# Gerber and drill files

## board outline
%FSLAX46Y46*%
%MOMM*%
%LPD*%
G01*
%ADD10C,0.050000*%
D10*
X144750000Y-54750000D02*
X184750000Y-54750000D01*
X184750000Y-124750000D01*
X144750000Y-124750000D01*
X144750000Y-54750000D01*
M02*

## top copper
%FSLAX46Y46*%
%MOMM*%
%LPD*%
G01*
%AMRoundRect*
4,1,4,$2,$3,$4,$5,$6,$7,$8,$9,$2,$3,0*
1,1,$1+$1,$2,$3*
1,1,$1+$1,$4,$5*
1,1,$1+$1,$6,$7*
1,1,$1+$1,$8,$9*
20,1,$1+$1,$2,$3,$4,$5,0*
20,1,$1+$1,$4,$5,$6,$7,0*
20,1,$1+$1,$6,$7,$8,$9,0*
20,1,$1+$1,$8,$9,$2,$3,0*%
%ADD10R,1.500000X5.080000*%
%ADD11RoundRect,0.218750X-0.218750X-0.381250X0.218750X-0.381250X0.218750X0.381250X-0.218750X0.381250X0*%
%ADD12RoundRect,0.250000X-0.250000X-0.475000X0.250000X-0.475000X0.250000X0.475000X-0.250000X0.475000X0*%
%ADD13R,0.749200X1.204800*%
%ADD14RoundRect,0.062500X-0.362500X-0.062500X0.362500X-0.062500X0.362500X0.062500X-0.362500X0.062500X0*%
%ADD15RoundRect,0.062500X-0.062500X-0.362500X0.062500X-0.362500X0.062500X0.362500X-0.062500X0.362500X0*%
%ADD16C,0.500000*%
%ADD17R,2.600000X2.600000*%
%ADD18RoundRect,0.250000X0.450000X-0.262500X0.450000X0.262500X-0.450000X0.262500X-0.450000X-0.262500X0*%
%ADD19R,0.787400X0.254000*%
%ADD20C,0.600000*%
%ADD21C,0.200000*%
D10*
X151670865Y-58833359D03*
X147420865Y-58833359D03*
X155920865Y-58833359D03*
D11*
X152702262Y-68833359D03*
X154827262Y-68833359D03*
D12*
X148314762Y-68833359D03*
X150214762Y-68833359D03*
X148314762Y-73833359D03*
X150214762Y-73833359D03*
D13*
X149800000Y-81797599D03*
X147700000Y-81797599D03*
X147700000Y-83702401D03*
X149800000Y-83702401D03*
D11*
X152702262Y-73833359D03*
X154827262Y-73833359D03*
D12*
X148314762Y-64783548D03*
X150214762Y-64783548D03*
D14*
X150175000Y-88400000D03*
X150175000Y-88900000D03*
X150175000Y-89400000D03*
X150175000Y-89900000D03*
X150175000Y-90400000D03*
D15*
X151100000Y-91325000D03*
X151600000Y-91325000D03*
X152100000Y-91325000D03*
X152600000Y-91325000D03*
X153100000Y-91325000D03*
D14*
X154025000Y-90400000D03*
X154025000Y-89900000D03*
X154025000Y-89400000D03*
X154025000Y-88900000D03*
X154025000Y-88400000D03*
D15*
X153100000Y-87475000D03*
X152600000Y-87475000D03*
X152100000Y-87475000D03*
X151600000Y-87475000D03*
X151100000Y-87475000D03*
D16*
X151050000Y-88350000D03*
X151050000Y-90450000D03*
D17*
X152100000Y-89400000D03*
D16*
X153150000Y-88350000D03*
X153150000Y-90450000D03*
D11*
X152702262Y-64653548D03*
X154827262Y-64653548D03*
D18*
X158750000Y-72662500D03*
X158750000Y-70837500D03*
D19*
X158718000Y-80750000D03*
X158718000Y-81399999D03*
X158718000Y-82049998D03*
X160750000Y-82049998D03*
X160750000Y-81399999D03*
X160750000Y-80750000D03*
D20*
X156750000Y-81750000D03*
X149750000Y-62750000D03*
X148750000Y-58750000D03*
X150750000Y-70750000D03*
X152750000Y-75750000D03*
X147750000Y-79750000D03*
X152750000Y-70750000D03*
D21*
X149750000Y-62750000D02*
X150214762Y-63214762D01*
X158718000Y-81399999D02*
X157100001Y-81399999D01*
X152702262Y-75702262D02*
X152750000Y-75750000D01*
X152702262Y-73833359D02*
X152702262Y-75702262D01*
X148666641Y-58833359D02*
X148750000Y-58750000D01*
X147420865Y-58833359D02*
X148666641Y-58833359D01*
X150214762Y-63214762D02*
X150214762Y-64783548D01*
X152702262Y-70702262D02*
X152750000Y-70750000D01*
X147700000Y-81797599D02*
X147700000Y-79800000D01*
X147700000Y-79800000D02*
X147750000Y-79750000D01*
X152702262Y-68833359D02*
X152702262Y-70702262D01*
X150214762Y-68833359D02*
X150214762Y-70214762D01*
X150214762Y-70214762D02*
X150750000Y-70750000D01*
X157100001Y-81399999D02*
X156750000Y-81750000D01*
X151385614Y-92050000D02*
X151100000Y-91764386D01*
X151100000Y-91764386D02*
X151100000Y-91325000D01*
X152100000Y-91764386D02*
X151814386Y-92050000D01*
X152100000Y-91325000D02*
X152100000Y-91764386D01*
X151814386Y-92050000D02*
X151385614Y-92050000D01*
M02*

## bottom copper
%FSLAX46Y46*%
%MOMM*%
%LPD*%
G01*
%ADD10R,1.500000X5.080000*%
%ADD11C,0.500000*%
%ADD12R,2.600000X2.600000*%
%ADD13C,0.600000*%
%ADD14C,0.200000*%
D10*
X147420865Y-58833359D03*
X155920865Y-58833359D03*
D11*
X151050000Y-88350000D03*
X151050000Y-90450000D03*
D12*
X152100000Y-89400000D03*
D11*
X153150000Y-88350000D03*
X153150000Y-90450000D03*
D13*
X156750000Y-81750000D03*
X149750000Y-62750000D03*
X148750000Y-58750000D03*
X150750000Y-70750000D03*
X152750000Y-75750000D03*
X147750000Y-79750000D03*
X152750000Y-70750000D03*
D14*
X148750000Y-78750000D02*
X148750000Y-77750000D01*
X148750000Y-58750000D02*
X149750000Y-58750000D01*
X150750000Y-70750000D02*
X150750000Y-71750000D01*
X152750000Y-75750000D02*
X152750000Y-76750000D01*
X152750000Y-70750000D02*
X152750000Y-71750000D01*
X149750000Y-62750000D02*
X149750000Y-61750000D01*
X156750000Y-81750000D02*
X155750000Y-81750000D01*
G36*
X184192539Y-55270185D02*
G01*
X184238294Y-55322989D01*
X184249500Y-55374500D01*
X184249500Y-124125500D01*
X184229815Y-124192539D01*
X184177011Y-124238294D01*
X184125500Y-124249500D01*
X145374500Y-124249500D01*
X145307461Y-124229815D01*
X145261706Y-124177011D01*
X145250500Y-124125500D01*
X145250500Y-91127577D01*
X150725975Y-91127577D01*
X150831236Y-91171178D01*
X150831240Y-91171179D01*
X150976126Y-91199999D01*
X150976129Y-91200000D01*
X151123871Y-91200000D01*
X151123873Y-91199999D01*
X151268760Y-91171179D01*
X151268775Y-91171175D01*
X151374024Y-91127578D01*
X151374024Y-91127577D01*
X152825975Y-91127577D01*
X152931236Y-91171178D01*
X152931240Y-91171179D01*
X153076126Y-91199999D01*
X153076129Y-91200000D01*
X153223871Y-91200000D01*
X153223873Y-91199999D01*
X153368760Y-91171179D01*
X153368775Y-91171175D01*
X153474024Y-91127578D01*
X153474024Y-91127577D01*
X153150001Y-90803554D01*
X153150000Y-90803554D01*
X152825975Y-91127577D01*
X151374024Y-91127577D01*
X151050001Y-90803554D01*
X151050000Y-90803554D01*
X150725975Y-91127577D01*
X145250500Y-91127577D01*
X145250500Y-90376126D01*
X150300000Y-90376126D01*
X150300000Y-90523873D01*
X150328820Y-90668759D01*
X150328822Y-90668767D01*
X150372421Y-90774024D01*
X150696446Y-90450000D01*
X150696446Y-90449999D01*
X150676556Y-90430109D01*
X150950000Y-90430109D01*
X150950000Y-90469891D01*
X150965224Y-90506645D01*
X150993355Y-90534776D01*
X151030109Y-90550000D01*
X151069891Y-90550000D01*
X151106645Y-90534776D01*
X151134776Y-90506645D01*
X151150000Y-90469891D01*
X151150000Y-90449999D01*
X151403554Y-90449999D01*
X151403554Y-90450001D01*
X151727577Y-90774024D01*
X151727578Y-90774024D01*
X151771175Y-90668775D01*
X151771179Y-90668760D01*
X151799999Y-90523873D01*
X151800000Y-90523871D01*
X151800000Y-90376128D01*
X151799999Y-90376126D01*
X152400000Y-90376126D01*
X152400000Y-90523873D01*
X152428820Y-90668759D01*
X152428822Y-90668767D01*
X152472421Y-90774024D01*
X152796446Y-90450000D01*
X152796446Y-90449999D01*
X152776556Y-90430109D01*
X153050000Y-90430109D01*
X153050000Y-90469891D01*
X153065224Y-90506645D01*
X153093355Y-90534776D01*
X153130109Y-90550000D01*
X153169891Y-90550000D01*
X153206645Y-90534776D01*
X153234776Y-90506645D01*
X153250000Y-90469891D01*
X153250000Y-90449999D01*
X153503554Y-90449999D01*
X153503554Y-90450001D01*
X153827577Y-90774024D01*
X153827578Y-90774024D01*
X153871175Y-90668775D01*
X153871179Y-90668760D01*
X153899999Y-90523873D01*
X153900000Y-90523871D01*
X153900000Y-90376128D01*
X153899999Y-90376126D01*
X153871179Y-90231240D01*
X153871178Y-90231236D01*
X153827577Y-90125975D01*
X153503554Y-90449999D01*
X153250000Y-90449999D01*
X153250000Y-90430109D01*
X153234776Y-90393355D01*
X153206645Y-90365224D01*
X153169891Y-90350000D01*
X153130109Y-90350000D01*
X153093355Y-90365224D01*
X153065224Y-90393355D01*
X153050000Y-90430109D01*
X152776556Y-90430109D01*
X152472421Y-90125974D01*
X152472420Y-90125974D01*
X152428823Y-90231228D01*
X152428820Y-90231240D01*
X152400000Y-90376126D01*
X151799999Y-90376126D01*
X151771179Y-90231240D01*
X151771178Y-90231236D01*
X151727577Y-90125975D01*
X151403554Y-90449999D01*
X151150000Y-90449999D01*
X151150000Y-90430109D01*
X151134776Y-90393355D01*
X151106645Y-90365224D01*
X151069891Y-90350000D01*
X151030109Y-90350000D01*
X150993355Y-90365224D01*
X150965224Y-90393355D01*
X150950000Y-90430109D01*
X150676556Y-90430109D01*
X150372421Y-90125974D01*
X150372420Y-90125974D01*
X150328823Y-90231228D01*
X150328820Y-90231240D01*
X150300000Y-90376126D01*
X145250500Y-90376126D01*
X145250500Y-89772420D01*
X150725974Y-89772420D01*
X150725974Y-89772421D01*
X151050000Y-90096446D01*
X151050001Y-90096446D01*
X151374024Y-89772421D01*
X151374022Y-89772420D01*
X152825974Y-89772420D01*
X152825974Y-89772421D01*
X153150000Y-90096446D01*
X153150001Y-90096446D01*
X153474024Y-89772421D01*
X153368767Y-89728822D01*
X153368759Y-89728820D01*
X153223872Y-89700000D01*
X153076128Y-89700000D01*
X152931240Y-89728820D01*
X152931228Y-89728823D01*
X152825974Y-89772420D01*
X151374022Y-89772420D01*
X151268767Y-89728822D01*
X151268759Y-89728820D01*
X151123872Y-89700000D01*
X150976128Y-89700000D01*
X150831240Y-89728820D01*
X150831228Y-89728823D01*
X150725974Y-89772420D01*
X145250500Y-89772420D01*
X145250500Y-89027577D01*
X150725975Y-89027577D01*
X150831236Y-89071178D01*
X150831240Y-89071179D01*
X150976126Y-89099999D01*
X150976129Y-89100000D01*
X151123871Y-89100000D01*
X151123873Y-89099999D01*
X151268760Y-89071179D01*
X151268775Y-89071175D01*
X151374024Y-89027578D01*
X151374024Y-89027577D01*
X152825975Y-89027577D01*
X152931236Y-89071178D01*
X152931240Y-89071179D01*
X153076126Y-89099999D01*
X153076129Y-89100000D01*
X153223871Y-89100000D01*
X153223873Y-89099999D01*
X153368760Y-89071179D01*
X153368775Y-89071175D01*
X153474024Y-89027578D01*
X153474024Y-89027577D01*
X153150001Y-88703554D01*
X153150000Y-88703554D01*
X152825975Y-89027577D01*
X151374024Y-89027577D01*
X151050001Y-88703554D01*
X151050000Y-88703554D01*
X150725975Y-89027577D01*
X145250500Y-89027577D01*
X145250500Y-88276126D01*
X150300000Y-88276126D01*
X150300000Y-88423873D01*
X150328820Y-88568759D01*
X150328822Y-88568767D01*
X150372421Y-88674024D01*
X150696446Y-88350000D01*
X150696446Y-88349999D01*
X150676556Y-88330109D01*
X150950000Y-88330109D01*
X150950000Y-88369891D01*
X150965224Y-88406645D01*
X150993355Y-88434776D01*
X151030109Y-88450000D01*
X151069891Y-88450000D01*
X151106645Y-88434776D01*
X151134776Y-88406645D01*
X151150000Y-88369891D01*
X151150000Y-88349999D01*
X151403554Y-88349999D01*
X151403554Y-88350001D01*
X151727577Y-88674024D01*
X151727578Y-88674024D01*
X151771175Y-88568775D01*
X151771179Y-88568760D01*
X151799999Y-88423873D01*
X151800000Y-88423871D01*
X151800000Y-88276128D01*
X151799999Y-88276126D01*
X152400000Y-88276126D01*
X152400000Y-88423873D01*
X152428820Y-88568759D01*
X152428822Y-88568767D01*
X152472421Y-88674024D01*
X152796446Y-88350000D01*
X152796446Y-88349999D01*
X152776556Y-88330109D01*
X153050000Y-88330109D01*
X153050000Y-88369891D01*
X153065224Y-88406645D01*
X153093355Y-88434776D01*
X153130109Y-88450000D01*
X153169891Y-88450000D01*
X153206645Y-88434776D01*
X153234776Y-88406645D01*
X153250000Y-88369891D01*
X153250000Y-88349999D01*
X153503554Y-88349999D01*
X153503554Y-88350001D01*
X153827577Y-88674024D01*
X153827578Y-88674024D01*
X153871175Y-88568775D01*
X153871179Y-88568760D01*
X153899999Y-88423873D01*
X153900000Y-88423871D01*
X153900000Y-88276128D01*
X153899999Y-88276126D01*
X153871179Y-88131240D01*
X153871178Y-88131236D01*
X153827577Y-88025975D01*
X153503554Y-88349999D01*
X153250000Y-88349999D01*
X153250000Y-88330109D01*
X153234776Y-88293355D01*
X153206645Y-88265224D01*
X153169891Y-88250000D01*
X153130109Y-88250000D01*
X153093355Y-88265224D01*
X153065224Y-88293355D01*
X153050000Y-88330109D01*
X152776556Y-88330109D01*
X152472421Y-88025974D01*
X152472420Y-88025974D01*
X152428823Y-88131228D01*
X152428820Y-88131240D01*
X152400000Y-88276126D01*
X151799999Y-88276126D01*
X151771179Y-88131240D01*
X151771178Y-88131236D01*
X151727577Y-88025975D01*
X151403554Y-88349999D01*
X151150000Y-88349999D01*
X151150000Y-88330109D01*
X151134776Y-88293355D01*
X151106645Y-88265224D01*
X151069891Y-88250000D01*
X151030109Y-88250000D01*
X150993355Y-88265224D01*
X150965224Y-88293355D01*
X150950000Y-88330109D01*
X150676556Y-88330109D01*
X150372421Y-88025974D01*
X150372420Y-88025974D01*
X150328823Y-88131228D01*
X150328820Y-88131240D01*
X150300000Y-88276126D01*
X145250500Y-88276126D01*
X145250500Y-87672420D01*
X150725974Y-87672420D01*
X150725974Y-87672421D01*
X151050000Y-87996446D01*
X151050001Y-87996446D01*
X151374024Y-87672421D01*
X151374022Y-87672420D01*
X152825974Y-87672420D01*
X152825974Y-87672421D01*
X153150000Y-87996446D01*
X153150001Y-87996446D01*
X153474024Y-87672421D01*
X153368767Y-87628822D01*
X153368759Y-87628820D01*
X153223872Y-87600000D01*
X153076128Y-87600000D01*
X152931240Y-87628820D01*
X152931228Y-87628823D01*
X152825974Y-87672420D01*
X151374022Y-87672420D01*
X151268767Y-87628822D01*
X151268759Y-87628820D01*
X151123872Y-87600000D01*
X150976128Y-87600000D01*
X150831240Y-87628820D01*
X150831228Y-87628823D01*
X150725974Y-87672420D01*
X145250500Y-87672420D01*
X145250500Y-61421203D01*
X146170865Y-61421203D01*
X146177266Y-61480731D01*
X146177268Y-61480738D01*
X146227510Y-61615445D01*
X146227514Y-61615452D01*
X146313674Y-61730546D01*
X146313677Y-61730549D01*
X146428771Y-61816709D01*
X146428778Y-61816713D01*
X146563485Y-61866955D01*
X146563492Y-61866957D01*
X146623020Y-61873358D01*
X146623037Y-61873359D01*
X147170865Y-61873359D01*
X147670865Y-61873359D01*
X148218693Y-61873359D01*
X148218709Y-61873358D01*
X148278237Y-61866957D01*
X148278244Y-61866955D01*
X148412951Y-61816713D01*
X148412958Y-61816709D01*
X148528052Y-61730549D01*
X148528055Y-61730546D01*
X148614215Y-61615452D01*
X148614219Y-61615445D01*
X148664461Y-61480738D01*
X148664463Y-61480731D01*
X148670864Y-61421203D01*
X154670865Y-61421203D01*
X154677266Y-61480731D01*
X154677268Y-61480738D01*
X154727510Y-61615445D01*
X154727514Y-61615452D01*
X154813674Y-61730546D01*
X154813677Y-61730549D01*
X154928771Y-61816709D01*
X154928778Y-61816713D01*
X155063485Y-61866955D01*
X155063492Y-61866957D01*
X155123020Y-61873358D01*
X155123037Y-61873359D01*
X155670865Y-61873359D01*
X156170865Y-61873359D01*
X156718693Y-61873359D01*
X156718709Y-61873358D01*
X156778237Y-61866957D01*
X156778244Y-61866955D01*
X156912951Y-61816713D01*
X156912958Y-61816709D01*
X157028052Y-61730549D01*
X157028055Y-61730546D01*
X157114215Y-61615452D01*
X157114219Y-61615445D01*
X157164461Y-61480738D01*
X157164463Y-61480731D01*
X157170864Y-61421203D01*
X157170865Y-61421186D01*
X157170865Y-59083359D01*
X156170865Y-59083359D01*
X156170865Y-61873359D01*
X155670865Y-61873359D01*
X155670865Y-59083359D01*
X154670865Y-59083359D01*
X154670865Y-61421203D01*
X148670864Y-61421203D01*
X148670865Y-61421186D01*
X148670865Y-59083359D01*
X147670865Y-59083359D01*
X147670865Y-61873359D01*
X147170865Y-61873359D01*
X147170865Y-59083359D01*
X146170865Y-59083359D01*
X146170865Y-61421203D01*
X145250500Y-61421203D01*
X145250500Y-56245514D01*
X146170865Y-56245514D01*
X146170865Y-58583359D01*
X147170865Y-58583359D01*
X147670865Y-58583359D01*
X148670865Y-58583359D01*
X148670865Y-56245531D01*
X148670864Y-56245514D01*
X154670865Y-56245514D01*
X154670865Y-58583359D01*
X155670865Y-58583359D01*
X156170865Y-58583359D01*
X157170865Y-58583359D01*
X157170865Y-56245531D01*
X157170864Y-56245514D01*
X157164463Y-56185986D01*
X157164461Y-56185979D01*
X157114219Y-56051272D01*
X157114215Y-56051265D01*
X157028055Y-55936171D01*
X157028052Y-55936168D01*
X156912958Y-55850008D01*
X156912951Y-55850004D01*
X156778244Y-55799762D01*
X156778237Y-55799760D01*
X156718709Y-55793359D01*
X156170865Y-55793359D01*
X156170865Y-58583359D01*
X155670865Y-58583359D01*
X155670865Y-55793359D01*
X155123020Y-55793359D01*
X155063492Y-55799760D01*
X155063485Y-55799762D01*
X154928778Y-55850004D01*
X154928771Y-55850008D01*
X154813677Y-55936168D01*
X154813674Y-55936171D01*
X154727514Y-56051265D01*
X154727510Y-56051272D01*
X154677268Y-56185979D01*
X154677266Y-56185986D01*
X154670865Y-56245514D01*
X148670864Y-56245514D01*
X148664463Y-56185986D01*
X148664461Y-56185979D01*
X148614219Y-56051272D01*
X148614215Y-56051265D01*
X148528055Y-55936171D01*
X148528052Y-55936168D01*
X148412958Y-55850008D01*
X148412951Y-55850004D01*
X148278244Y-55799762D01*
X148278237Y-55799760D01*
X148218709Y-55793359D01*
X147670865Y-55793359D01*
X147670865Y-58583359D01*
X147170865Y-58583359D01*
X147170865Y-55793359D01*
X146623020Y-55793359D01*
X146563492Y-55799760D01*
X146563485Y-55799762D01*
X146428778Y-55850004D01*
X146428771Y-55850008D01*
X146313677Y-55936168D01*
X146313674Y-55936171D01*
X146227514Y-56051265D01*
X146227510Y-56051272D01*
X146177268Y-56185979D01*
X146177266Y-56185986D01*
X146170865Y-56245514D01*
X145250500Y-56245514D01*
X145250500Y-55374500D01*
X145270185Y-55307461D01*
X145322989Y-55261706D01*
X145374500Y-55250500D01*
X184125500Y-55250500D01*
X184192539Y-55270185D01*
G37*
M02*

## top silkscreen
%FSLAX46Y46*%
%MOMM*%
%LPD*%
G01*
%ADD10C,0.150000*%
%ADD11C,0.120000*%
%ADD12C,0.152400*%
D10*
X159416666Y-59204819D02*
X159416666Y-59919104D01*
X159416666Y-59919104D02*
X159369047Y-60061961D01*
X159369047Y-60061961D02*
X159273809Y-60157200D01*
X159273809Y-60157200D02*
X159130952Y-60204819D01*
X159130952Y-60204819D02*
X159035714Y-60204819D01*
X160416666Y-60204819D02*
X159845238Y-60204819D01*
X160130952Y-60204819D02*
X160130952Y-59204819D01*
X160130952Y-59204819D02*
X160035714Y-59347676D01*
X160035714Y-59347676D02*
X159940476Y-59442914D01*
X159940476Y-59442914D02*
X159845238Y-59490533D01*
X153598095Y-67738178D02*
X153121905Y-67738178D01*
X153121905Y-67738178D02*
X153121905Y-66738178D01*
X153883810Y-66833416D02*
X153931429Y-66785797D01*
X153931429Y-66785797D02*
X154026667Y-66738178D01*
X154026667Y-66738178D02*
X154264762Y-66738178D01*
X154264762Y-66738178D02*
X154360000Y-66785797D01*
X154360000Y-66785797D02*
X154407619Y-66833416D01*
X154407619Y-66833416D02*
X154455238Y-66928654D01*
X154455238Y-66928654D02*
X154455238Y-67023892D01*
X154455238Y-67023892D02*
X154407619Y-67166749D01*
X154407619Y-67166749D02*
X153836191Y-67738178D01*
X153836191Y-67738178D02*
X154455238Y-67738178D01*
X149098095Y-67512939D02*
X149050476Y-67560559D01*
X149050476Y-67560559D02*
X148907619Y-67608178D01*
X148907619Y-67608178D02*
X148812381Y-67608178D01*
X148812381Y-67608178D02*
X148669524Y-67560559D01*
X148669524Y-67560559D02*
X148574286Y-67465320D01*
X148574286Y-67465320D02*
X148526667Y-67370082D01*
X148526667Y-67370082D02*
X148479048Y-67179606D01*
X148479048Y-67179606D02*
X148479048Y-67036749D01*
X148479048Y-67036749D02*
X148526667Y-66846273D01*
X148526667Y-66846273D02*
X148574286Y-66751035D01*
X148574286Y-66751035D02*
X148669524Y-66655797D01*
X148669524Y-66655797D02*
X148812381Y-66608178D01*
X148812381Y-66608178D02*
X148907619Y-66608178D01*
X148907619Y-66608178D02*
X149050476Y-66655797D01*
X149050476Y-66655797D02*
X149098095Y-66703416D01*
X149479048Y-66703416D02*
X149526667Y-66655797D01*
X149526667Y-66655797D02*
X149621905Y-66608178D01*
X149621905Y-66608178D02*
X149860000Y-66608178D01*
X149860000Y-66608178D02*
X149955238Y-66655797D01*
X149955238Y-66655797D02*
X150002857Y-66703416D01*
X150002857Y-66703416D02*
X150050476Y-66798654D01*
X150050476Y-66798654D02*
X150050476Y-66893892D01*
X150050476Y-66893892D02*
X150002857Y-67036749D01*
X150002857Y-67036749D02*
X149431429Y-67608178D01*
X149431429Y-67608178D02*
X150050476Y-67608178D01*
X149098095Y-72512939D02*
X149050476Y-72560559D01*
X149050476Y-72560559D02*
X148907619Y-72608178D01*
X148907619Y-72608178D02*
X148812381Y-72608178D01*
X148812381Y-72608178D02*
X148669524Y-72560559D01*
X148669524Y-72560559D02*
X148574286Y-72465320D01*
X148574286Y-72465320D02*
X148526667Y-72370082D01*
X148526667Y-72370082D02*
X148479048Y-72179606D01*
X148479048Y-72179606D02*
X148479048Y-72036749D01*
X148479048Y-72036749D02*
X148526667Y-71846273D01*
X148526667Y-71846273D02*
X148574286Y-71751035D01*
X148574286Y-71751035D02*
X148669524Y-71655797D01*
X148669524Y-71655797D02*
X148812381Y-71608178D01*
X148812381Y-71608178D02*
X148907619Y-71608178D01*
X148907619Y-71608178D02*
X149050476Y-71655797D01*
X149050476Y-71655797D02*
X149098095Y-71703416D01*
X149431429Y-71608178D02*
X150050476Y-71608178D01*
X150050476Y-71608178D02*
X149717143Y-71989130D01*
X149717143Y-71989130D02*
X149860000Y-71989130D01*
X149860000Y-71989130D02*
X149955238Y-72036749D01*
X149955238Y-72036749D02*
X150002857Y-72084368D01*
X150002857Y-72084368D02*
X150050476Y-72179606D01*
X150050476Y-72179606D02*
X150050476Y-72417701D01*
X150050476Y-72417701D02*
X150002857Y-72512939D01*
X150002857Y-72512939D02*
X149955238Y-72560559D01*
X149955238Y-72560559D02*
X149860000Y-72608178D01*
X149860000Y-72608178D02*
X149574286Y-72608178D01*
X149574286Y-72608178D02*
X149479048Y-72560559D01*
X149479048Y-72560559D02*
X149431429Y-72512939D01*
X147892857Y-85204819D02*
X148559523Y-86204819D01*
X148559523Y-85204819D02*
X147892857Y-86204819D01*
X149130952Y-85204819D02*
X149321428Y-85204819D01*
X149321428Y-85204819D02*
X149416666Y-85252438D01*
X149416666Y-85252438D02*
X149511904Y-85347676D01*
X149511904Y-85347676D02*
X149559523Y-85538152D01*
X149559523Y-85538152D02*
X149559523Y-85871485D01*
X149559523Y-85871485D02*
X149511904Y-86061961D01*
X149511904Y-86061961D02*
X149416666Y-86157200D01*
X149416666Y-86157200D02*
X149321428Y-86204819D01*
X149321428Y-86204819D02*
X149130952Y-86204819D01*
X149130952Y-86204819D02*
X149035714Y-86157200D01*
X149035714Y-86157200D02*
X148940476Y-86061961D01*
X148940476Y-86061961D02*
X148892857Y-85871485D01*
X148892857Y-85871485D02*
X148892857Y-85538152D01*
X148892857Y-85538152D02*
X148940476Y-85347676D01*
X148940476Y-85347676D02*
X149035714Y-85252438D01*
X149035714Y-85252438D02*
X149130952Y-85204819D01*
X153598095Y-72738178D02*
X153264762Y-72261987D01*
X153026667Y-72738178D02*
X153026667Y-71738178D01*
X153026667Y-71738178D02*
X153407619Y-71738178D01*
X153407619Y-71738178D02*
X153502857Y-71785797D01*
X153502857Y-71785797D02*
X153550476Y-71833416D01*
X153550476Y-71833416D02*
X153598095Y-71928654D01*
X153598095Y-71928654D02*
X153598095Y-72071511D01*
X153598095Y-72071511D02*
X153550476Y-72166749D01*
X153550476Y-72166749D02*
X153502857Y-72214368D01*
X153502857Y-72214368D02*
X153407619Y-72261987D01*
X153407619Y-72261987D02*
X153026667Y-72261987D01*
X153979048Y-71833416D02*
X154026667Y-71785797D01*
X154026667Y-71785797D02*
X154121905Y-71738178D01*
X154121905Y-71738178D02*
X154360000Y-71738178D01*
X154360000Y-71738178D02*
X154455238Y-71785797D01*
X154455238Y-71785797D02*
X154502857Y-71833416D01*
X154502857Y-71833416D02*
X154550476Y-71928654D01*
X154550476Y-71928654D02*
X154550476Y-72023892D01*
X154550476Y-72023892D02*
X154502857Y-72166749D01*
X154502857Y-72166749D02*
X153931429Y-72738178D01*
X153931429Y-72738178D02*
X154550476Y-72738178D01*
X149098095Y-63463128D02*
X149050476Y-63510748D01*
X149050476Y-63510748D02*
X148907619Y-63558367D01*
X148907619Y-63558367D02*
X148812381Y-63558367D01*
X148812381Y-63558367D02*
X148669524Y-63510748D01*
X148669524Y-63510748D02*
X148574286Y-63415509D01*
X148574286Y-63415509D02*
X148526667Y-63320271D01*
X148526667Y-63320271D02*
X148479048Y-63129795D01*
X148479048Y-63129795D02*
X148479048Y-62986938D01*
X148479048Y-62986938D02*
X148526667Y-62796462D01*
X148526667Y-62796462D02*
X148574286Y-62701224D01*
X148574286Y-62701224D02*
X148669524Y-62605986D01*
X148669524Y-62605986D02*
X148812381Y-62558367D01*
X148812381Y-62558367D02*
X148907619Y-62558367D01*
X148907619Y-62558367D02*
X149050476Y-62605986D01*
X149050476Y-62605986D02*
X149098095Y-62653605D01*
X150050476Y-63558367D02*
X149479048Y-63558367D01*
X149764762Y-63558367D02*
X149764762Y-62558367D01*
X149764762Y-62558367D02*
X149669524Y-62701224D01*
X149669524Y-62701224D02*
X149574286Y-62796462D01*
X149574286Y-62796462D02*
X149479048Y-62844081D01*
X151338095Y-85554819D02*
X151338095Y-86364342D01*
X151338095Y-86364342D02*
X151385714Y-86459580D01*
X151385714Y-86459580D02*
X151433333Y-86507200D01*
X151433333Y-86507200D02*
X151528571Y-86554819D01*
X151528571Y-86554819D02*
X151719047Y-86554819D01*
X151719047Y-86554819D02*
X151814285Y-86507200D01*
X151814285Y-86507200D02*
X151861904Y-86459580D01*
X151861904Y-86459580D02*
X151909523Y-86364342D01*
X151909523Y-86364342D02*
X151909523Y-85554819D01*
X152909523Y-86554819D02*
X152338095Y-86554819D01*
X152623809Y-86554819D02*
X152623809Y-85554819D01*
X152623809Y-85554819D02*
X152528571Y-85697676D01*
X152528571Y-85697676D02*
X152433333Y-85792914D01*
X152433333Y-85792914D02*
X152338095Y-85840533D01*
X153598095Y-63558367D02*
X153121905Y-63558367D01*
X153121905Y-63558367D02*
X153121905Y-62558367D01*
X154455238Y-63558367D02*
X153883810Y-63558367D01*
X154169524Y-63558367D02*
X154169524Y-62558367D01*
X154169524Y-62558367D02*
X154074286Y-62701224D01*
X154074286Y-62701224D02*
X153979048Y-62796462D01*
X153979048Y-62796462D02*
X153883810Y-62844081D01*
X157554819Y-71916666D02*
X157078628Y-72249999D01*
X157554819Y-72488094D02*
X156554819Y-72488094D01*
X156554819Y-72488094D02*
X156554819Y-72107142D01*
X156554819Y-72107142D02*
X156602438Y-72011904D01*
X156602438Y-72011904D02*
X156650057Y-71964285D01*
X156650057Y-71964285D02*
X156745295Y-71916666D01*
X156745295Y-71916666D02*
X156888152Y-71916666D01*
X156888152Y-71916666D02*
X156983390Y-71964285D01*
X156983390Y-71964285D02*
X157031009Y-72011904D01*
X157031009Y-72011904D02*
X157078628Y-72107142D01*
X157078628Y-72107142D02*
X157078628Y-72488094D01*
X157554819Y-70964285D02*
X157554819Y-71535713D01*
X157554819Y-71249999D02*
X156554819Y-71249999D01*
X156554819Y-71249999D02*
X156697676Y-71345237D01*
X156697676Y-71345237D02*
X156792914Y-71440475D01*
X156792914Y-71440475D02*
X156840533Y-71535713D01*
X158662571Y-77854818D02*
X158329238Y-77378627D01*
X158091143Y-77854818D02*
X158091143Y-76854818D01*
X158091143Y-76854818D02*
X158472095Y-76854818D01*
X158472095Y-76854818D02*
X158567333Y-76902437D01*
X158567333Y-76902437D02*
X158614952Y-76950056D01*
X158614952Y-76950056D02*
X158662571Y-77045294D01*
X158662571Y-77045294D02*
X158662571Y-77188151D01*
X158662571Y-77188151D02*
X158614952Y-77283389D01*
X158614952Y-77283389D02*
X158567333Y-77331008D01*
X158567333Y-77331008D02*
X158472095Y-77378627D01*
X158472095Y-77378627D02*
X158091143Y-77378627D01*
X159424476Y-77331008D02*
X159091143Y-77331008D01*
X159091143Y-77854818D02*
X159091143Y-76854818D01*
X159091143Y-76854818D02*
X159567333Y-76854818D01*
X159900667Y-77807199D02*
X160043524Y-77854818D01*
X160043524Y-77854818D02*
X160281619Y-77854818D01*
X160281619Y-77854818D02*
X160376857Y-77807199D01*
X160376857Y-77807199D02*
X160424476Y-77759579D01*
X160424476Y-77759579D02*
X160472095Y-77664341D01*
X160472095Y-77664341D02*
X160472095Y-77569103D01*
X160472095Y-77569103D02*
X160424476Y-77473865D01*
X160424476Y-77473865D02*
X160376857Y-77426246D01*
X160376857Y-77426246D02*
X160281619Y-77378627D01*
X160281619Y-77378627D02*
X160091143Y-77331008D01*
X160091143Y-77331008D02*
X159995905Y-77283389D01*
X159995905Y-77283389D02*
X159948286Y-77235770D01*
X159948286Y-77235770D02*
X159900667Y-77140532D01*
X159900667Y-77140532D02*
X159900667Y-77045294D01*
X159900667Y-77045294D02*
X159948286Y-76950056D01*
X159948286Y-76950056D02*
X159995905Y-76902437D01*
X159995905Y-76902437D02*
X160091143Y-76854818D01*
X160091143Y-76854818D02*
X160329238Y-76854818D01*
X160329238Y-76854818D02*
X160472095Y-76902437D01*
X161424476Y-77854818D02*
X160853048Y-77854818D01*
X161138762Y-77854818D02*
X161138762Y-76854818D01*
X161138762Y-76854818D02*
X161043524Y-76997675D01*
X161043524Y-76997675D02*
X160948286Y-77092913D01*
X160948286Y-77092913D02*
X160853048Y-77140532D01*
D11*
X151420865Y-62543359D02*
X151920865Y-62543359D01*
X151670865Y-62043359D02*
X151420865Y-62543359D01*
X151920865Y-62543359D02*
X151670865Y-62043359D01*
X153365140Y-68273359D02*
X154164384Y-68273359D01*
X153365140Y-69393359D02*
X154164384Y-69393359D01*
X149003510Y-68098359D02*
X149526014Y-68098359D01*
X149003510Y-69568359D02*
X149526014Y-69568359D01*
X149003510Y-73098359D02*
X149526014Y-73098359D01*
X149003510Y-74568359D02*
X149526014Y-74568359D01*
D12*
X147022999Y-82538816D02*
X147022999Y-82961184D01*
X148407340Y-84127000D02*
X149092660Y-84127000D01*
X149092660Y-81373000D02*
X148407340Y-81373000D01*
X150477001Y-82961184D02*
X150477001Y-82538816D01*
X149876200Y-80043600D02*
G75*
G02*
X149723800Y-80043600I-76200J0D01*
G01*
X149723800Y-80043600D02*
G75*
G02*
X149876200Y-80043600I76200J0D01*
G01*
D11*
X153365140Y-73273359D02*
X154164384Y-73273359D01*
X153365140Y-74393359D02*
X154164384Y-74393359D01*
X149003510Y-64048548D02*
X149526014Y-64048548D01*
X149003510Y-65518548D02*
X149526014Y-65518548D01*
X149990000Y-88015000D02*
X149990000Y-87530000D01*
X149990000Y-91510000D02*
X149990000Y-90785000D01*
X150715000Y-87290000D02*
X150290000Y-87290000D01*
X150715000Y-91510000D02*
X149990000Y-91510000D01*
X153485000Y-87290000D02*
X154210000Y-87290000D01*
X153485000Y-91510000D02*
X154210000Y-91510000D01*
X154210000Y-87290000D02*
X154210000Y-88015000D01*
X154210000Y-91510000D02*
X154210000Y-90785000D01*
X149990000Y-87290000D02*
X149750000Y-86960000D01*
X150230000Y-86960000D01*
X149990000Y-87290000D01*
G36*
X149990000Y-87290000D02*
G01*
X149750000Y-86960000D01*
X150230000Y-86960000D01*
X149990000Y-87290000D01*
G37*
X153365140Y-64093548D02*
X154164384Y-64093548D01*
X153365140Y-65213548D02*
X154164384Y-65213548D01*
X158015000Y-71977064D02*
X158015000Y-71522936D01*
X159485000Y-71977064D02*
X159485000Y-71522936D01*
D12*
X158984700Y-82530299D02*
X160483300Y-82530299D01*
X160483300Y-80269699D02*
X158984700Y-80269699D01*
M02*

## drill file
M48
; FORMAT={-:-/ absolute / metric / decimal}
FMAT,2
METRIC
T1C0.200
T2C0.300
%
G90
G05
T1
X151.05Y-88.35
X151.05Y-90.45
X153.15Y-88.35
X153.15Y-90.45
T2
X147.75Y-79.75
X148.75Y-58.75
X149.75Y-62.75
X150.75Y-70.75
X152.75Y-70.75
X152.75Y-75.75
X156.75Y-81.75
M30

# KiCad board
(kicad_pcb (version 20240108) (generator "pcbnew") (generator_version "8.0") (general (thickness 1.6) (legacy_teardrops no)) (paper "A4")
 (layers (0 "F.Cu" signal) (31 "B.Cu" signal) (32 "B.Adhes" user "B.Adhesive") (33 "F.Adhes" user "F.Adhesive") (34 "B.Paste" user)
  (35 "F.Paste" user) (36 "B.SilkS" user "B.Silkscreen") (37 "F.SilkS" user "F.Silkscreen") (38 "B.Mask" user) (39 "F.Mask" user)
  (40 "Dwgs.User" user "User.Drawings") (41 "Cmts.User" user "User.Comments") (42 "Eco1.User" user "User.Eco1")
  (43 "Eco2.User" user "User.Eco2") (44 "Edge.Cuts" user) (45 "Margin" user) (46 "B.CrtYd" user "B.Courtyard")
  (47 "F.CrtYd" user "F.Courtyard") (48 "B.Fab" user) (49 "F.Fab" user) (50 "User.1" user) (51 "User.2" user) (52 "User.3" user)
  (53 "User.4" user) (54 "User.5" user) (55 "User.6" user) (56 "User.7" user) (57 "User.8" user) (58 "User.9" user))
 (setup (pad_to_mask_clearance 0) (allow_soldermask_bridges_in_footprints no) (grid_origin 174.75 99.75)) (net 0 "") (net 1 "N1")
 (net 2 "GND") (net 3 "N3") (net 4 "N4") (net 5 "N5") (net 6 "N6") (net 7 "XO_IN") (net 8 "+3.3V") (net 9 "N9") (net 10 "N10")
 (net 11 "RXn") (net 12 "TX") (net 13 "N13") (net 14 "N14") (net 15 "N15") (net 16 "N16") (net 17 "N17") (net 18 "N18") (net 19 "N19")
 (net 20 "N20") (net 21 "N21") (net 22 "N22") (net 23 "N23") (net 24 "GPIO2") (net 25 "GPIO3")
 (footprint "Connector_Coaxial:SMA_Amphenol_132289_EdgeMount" (layer "F.Cu") (at 151.670865 58.833359 90)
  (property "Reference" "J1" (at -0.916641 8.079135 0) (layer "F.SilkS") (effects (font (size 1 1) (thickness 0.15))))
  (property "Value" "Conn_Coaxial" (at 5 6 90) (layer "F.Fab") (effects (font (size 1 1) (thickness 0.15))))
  (fp_line (start -3.71 -0.25) (end -3.71 0.25) (stroke (width 0.12) (type solid)) (layer "F.SilkS"))
  (fp_line (start -3.21 0) (end -3.71 -0.25) (stroke (width 0.12) (type solid)) (layer "F.SilkS"))
  (fp_line (start -3.71 0.25) (end -3.21 0) (stroke (width 0.12) (type solid)) (layer "F.SilkS"))
  (pad "1" smd rect (at 0 0 180) (size 1.5 5.08) (layers "F.Cu" "F.Paste" "F.Mask") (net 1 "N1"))
  (pad "2" smd rect (at 0 -4.25 180) (size 1.5 5.08) (layers "F.Cu" "F.Paste" "F.Mask") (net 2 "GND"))
  (pad "2" smd rect (at 0 -4.25 180) (size 1.5 5.08) (layers "B.Cu" "B.Paste" "B.Mask") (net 2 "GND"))
  (pad "2" smd rect (at 0 4.25 180) (size 1.5 5.08) (layers "F.Cu" "F.Paste" "F.Mask") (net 2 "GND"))
  (pad "2" smd rect (at 0 4.25 180) (size 1.5 5.08) (layers "B.Cu" "B.Paste" "B.Mask") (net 2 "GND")))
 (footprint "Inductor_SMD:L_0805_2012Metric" (layer "F.Cu") (at 153.764762 68.833359)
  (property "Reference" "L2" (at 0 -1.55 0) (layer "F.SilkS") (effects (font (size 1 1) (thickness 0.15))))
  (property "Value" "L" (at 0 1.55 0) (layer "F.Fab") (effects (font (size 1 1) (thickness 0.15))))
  (fp_line (start -0.399622 -0.56) (end 0.399622 -0.56) (stroke (width 0.12) (type solid)) (layer "F.SilkS"))
  (fp_line (start -0.399622 0.56) (end 0.399622 0.56) (stroke (width 0.12) (type solid)) (layer "F.SilkS"))
  (pad "1" smd roundrect (at -1.0625 0) (size 0.875 1.2) (layers "F.Cu" "F.Paste" "F.Mask") (roundrect_rratio 0.25) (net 2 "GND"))
  (pad "2" smd roundrect (at 1.0625 0) (size 0.875 1.2) (layers "F.Cu" "F.Paste" "F.Mask") (roundrect_rratio 0.25) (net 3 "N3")))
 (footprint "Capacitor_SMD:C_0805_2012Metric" (layer "F.Cu") (at 149.264762 68.833359)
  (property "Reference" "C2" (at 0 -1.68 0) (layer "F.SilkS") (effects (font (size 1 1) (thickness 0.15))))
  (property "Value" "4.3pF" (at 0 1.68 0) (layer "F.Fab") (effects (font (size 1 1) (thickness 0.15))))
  (fp_line (start -0.261252 -0.735) (end 0.261252 -0.735) (stroke (width 0.12) (type solid)) (layer "F.SilkS"))
  (fp_line (start -0.261252 0.735) (end 0.261252 0.735) (stroke (width 0.12) (type solid)) (layer "F.SilkS"))
  (pad "1" smd roundrect (at -0.95 0) (size 1 1.45) (layers "F.Cu" "F.Paste" "F.Mask") (roundrect_rratio 0.25) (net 1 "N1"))
  (pad "2" smd roundrect (at 0.95 0) (size 1 1.45) (layers "F.Cu" "F.Paste" "F.Mask") (roundrect_rratio 0.25) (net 2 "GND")))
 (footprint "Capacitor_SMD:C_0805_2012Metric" (layer "F.Cu") (at 149.264762 73.833359)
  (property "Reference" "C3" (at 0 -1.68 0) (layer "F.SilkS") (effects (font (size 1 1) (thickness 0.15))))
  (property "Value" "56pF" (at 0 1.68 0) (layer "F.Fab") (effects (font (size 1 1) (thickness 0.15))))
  (fp_line (start -0.261252 -0.735) (end 0.261252 -0.735) (stroke (width 0.12) (type solid)) (layer "F.SilkS"))
  (fp_line (start -0.261252 0.735) (end 0.261252 0.735) (stroke (width 0.12) (type solid)) (layer "F.SilkS"))
  (pad "1" smd roundrect (at -0.95 0) (size 1 1.45) (layers "F.Cu" "F.Paste" "F.Mask") (roundrect_rratio 0.25) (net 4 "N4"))
  (pad "2" smd roundrect (at 0.95 0) (size 1 1.45) (layers "F.Cu" "F.Paste" "F.Mask") (roundrect_rratio 0.25) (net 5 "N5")))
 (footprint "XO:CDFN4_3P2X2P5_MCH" (layer "F.Cu") (at 148.75 82.75 -90)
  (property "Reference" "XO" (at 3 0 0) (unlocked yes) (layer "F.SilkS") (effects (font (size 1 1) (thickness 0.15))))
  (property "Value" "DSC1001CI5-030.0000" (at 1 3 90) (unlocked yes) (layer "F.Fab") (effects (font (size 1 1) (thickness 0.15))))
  (fp_line (start -0.211184 1.727001) (end 0.211184 1.727001) (stroke (width 0.1524) (type solid)) (layer "F.SilkS"))
  (fp_line (start 1.377 0.34266) (end 1.377 -0.34266) (stroke (width 0.1524) (type solid)) (layer "F.SilkS"))
  (fp_line (start -1.377 -0.34266) (end -1.377 0.34266) (stroke (width 0.1524) (type solid)) (layer "F.SilkS"))
  (fp_line (start 0.211184 -1.727001) (end -0.211184 -1.727001) (stroke (width 0.1524) (type solid)) (layer "F.SilkS"))
  (fp_circle (center -2.7064 -1.05) (end -2.6302 -1.05) (stroke (width 0.1524) (type solid)) (fill none) (layer "F.SilkS"))
  (pad "1" smd rect (at -0.952401 -1.05 270) (size 1.2048 0.7492) (layers "F.Cu" "F.Paste" "F.Mask") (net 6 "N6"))
  (pad "2" smd rect (at -0.952401 1.05 270) (size 1.2048 0.7492) (layers "F.Cu" "F.Paste" "F.Mask") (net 2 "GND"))
  (pad "3" smd rect (at 0.952401 1.05 270) (size 1.2048 0.7492) (layers "F.Cu" "F.Paste" "F.Mask") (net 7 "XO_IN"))
  (pad "4" smd rect (at 0.952401 -1.05 270) (size 1.2048 0.7492) (layers "F.Cu" "F.Paste" "F.Mask") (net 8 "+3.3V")))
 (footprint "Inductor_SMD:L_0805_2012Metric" (layer "F.Cu") (at 153.764762 73.833359)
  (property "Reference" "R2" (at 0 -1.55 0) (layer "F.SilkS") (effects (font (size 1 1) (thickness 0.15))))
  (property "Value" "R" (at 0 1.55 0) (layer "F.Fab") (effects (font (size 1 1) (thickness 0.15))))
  (fp_line (start -0.399622 -0.56) (end 0.399622 -0.56) (stroke (width 0.12) (type solid)) (layer "F.SilkS"))
  (fp_line (start -0.399622 0.56) (end 0.399622 0.56) (stroke (width 0.12) (type solid)) (layer "F.SilkS"))
  (pad "1" smd roundrect (at -1.0625 0) (size 0.875 1.2) (layers "F.Cu" "F.Paste" "F.Mask") (roundrect_rratio 0.25) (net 2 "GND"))
  (pad "2" smd roundrect (at 1.0625 0) (size 0.875 1.2) (layers "F.Cu" "F.Paste" "F.Mask") (roundrect_rratio 0.25) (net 4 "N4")))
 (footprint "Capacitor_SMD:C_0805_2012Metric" (layer "F.Cu") (at 149.264762 64.783548)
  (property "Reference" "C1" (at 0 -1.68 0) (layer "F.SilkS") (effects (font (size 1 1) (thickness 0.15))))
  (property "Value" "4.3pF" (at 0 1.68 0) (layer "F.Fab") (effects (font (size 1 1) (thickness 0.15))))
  (fp_line (start -0.261252 -0.735) (end 0.261252 -0.735) (stroke (width 0.12) (type solid)) (layer "F.SilkS"))
  (fp_line (start -0.261252 0.735) (end 0.261252 0.735) (stroke (width 0.12) (type solid)) (layer "F.SilkS"))
  (pad "1" smd roundrect (at -0.95 0) (size 1 1.45) (layers "F.Cu" "F.Paste" "F.Mask") (roundrect_rratio 0.25) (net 5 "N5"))
  (pad "2" smd roundrect (at 0.95 0) (size 1 1.45) (layers "F.Cu" "F.Paste" "F.Mask") (roundrect_rratio 0.25) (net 2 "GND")))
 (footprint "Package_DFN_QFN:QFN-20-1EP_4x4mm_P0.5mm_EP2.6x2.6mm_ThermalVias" (layer "F.Cu") (at 152.1 89.4)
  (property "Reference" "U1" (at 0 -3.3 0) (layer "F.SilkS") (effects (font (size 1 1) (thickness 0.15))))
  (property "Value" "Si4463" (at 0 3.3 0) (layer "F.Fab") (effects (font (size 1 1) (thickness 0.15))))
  (fp_line (start -2.11 -1.385) (end -2.11 -1.87) (stroke (width 0.12) (type solid)) (layer "F.SilkS"))
  (fp_line (start -2.11 2.11) (end -2.11 1.385) (stroke (width 0.12) (type solid)) (layer "F.SilkS"))
  (fp_line (start -1.385 -2.11) (end -1.81 -2.11) (stroke (width 0.12) (type solid)) (layer "F.SilkS"))
  (fp_line (start -1.385 2.11) (end -2.11 2.11) (stroke (width 0.12) (type solid)) (layer "F.SilkS"))
  (fp_line (start 1.385 -2.11) (end 2.11 -2.11) (stroke (width 0.12) (type solid)) (layer "F.SilkS"))
  (fp_line (start 1.385 2.11) (end 2.11 2.11) (stroke (width 0.12) (type solid)) (layer "F.SilkS"))
  (fp_line (start 2.11 -2.11) (end 2.11 -1.385) (stroke (width 0.12) (type solid)) (layer "F.SilkS"))
  (fp_line (start 2.11 2.11) (end 2.11 1.385) (stroke (width 0.12) (type solid)) (layer "F.SilkS"))
  (fp_poly
   (pts (xy -2.11 -2.11) (xy -2.35 -2.44) (xy -1.87 -2.44) (xy -2.11 -2.11)) (stroke (width 0.12) (type solid)) (fill solid)
   (layer "F.SilkS"))
  (pad "" smd roundrect (at -0.65 -0.65) (size 1.13 1.13) (layers "F.Paste") (roundrect_rratio 0.221239))
  (pad "" smd roundrect (at -0.65 0.65) (size 1.13 1.13) (layers "F.Paste") (roundrect_rratio 0.221239))
  (pad "" smd roundrect (at 0.65 -0.65) (size 1.13 1.13) (layers "F.Paste") (roundrect_rratio 0.221239))
  (pad "" smd roundrect (at 0.65 0.65) (size 1.13 1.13) (layers "F.Paste") (roundrect_rratio 0.221239))
  (pad "1" smd roundrect (at -1.925 -1) (size 0.85 0.25) (layers "F.Cu" "F.Paste" "F.Mask") (roundrect_rratio 0.25) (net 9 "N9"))
  (pad "2" smd roundrect (at -1.925 -0.5) (size 0.85 0.25) (layers "F.Cu" "F.Paste" "F.Mask") (roundrect_rratio 0.25) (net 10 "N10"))
  (pad "3" smd roundrect (at -1.925 0) (size 0.85 0.25) (layers "F.Cu" "F.Paste" "F.Mask") (roundrect_rratio 0.25) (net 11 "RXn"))
  (pad "4" smd roundrect (at -1.925 0.5) (size 0.85 0.25) (layers "F.Cu" "F.Paste" "F.Mask") (roundrect_rratio 0.25) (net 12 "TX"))
  (pad "5" smd roundrect (at -1.925 1) (size 0.85 0.25) (layers "F.Cu" "F.Paste" "F.Mask") (roundrect_rratio 0.25) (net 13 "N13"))
  (pad "6" smd roundrect (at -1 1.925) (size 0.25 0.85) (layers "F.Cu" "F.Paste" "F.Mask") (roundrect_rratio 0.25) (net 8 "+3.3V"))
  (pad "7" smd roundrect (at -0.5 1.925) (size 0.25 0.85) (layers "F.Cu" "F.Paste" "F.Mask") (roundrect_rratio 0.25) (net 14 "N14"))
  (pad "8" smd roundrect (at 0 1.925) (size 0.25 0.85) (layers "F.Cu" "F.Paste" "F.Mask") (roundrect_rratio 0.25) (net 8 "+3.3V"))
  (pad "9" smd roundrect (at 0.5 1.925) (size 0.25 0.85) (layers "F.Cu" "F.Paste" "F.Mask") (roundrect_rratio 0.25) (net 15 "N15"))
  (pad "10" smd roundrect (at 1 1.925) (size 0.25 0.85) (layers "F.Cu" "F.Paste" "F.Mask") (roundrect_rratio 0.25) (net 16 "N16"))
  (pad "11" smd roundrect (at 1.925 1) (size 0.85 0.25) (layers "F.Cu" "F.Paste" "F.Mask") (roundrect_rratio 0.25) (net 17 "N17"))
  (pad "12" smd roundrect (at 1.925 0.5) (size 0.85 0.25) (layers "F.Cu" "F.Paste" "F.Mask") (roundrect_rratio 0.25) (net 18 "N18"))
  (pad "13" smd roundrect (at 1.925 0) (size 0.85 0.25) (layers "F.Cu" "F.Paste" "F.Mask") (roundrect_rratio 0.25) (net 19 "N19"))
  (pad "14" smd roundrect (at 1.925 -0.5) (size 0.85 0.25) (layers "F.Cu" "F.Paste" "F.Mask") (roundrect_rratio 0.25) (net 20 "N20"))
  (pad "15" smd roundrect (at 1.925 -1) (size 0.85 0.25) (layers "F.Cu" "F.Paste" "F.Mask") (roundrect_rratio 0.25) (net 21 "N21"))
  (pad "16" smd roundrect (at 1 -1.925) (size 0.25 0.85) (layers "F.Cu" "F.Paste" "F.Mask") (roundrect_rratio 0.25) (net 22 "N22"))
  (pad "17" smd roundrect (at 0.5 -1.925) (size 0.25 0.85) (layers "F.Cu" "F.Paste" "F.Mask") (roundrect_rratio 0.25) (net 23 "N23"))
  (pad "18" smd roundrect (at 0 -1.925) (size 0.25 0.85) (layers "F.Cu" "F.Paste" "F.Mask") (roundrect_rratio 0.25) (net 2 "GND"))
  (pad "19" smd roundrect (at -0.5 -1.925) (size 0.25 0.85) (layers "F.Cu" "F.Paste" "F.Mask") (roundrect_rratio 0.25) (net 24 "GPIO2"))
  (pad "20" smd roundrect (at -1 -1.925) (size 0.25 0.85) (layers "F.Cu" "F.Paste" "F.Mask") (roundrect_rratio 0.25) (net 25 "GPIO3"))
  (pad "21" thru_hole circle (at -1.05 -1.05) (size 0.5 0.5) (drill 0.2) (layers "*.Cu") (remove_unused_layers no) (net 2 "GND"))
  (pad "21" thru_hole circle (at -1.05 1.05) (size 0.5 0.5) (drill 0.2) (layers "*.Cu") (remove_unused_layers no) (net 2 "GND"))
  (pad "21" smd rect (at 0 0) (size 2.6 2.6) (layers "F.Cu" "F.Mask") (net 2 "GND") (zone_connect 2))
  (pad "21" smd rect (at 0 0) (size 2.6 2.6) (layers "B.Cu") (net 2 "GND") (zone_connect 2))
  (pad "21" thru_hole circle (at 1.05 -1.05) (size 0.5 0.5) (drill 0.2) (layers "*.Cu") (remove_unused_layers no) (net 2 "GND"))
  (pad "21" thru_hole circle (at 1.05 1.05) (size 0.5 0.5) (drill 0.2) (layers "*.Cu") (remove_unused_layers no) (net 2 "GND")))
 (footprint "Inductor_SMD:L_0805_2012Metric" (layer "F.Cu") (at 153.764762 64.653548)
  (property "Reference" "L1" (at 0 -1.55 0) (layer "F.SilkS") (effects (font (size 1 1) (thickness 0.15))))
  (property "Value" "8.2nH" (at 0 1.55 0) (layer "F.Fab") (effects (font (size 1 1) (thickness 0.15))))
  (fp_line (start -0.399622 -0.56) (end 0.399622 -0.56) (stroke (width 0.12) (type solid)) (layer "F.SilkS"))
  (fp_line (start -0.399622 0.56) (end 0.399622 0.56) (stroke (width 0.12) (type solid)) (layer "F.SilkS"))
  (pad "1" smd roundrect (at -1.0625 0) (size 0.875 1.2) (layers "F.Cu" "F.Paste" "F.Mask") (roundrect_rratio 0.25) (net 5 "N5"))
  (pad "2" smd roundrect (at 1.0625 0) (size 0.875 1.2) (layers "F.Cu" "F.Paste" "F.Mask") (roundrect_rratio 0.25) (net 1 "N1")))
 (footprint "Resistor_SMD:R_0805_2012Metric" (layer "F.Cu") (at 158.75 71.75 90)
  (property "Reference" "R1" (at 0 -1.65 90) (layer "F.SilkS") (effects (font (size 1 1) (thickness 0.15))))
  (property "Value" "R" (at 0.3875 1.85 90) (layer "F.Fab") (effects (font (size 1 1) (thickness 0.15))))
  (fp_line (start -0.227064 -0.735) (end 0.227064 -0.735) (stroke (width 0.12) (type solid)) (layer "F.SilkS"))
  (fp_line (start -0.227064 0.735) (end 0.227064 0.735) (stroke (width 0.12) (type solid)) (layer "F.SilkS"))
  (pad "1" smd roundrect (at -0.9125 0 90) (size 1.025 1.4) (layers "F.Cu" "F.Paste" "F.Mask") (roundrect_rratio 0.243902) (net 4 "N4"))
  (pad "2" smd roundrect (at 0.9125 0 90) (size 1.025 1.4) (layers "F.Cu" "F.Paste" "F.Mask") (roundrect_rratio 0.243902) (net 3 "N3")))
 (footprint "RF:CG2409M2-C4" (layer "F.Cu") (at 159.734 81.399999)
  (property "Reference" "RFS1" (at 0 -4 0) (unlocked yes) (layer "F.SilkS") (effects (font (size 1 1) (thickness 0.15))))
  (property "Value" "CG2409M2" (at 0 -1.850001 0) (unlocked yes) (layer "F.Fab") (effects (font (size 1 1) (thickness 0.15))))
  (fp_line (start -0.7493 1.1303) (end 0.7493 1.1303) (stroke (width 0.1524) (type solid)) (layer "F.SilkS"))
  (fp_line (start 0.7493 -1.1303) (end -0.7493 -1.1303) (stroke (width 0.1524) (type solid)) (layer "F.SilkS"))
  (pad "1" smd rect (at -1.016 -0.649999) (size 0.7874 0.254) (layers "F.Cu" "F.Paste" "F.Mask") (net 11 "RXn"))
  (pad "2" smd rect (at -1.016 0) (size 0.7874 0.254) (layers "F.Cu" "F.Paste" "F.Mask") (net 2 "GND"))
  (pad "3" smd rect (at -1.016 0.649999) (size 0.7874 0.254) (layers "F.Cu" "F.Paste" "F.Mask") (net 12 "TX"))
  (pad "4" smd rect (at 1.016 0.649999) (size 0.7874 0.254) (layers "F.Cu" "F.Paste" "F.Mask") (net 24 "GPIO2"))
  (pad "5" smd rect (at 1.016 0) (size 0.7874 0.254) (layers "F.Cu" "F.Paste" "F.Mask") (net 3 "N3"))
  (pad "6" smd rect (at 1.016 -0.649999) (size 0.7874 0.254) (layers "F.Cu" "F.Paste" "F.Mask") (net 25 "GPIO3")))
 (gr_rect (start 144.75 54.75) (end 184.75 124.75) (stroke (width 0.05) (type default)) (fill none) (layer "Edge.Cuts"))
 (segment (start 149.75 62.75) (end 150.214762 63.214762) (width 0.2) (layer "F.Cu") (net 2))
 (segment (start 158.718 81.399999) (end 157.100001 81.399999) (width 0.2) (layer "F.Cu") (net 2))
 (segment (start 152.702262 75.702262) (end 152.75 75.75) (width 0.2) (layer "F.Cu") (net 2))
 (segment (start 152.702262 73.833359) (end 152.702262 75.702262) (width 0.2) (layer "F.Cu") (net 2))
 (segment (start 148.666641 58.833359) (end 148.75 58.75) (width 0.2) (layer "F.Cu") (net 2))
 (segment (start 147.420865 58.833359) (end 148.666641 58.833359) (width 0.2) (layer "F.Cu") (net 2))
 (segment (start 150.214762 63.214762) (end 150.214762 64.783548) (width 0.2) (layer "F.Cu") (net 2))
 (segment (start 152.702262 70.702262) (end 152.75 70.75) (width 0.2) (layer "F.Cu") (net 2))
 (segment (start 147.7 81.797599) (end 147.7 79.8) (width 0.2) (layer "F.Cu") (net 2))
 (segment (start 147.7 79.8) (end 147.75 79.75) (width 0.2) (layer "F.Cu") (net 2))
 (segment (start 152.702262 68.833359) (end 152.702262 70.702262) (width 0.2) (layer "F.Cu") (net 2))
 (segment (start 150.214762 68.833359) (end 150.214762 70.214762) (width 0.2) (layer "F.Cu") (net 2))
 (segment (start 150.214762 70.214762) (end 150.75 70.75) (width 0.2) (layer "F.Cu") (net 2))
 (segment (start 157.100001 81.399999) (end 156.75 81.75) (width 0.2) (layer "F.Cu") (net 2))
 (via (at 156.75 81.75) (size 0.6) (drill 0.3) (layers "F.Cu" "B.Cu") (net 2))
 (via (at 149.75 62.75) (size 0.6) (drill 0.3) (layers "F.Cu" "B.Cu") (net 2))
 (via (at 148.75 58.75) (size 0.6) (drill 0.3) (layers "F.Cu" "B.Cu") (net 2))
 (via (at 150.75 70.75) (size 0.6) (drill 0.3) (layers "F.Cu" "B.Cu") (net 2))
 (via (at 152.75 75.75) (size 0.6) (drill 0.3) (layers "F.Cu" "B.Cu") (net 2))
 (via (at 147.75 79.75) (size 0.6) (drill 0.3) (layers "F.Cu" "B.Cu") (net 2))
 (via (at 152.75 70.75) (size 0.6) (drill 0.3) (layers "F.Cu" "B.Cu") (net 2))
 (segment (start 148.75 78.75) (end 148.75 77.75) (width 0.2) (layer "B.Cu") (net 2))
 (segment (start 148.75 58.75) (end 149.75 58.75) (width 0.2) (layer "B.Cu") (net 2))
 (segment (start 150.75 70.75) (end 150.75 71.75) (width 0.2) (layer "B.Cu") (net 2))
 (segment (start 152.75 75.75) (end 152.75 76.75) (width 0.2) (layer "B.Cu") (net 2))
 (segment (start 152.75 70.75) (end 152.75 71.75) (width 0.2) (layer "B.Cu") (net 2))
 (segment (start 149.75 62.75) (end 149.75 61.75) (width 0.2) (layer "B.Cu") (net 2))
 (segment (start 156.75 81.75) (end 155.75 81.75) (width 0.2) (layer "B.Cu") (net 2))
 (segment (start 151.385614 92.05) (end 151.1 91.764386) (width 0.2) (layer "F.Cu") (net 8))
 (segment (start 151.1 91.764386) (end 151.1 91.325) (width 0.2) (layer "F.Cu") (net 8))
 (segment (start 152.1 91.764386) (end 151.814386 92.05) (width 0.2) (layer "F.Cu") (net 8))
 (segment (start 152.1 91.325) (end 152.1 91.764386) (width 0.2) (layer "F.Cu") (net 8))
 (segment (start 151.814386 92.05) (end 151.385614 92.05) (width 0.2) (layer "F.Cu") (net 8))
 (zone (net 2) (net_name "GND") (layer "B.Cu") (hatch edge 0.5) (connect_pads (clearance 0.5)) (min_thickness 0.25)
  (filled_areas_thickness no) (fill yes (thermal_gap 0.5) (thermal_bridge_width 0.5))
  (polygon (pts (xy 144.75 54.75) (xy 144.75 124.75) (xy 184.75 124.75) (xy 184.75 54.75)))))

